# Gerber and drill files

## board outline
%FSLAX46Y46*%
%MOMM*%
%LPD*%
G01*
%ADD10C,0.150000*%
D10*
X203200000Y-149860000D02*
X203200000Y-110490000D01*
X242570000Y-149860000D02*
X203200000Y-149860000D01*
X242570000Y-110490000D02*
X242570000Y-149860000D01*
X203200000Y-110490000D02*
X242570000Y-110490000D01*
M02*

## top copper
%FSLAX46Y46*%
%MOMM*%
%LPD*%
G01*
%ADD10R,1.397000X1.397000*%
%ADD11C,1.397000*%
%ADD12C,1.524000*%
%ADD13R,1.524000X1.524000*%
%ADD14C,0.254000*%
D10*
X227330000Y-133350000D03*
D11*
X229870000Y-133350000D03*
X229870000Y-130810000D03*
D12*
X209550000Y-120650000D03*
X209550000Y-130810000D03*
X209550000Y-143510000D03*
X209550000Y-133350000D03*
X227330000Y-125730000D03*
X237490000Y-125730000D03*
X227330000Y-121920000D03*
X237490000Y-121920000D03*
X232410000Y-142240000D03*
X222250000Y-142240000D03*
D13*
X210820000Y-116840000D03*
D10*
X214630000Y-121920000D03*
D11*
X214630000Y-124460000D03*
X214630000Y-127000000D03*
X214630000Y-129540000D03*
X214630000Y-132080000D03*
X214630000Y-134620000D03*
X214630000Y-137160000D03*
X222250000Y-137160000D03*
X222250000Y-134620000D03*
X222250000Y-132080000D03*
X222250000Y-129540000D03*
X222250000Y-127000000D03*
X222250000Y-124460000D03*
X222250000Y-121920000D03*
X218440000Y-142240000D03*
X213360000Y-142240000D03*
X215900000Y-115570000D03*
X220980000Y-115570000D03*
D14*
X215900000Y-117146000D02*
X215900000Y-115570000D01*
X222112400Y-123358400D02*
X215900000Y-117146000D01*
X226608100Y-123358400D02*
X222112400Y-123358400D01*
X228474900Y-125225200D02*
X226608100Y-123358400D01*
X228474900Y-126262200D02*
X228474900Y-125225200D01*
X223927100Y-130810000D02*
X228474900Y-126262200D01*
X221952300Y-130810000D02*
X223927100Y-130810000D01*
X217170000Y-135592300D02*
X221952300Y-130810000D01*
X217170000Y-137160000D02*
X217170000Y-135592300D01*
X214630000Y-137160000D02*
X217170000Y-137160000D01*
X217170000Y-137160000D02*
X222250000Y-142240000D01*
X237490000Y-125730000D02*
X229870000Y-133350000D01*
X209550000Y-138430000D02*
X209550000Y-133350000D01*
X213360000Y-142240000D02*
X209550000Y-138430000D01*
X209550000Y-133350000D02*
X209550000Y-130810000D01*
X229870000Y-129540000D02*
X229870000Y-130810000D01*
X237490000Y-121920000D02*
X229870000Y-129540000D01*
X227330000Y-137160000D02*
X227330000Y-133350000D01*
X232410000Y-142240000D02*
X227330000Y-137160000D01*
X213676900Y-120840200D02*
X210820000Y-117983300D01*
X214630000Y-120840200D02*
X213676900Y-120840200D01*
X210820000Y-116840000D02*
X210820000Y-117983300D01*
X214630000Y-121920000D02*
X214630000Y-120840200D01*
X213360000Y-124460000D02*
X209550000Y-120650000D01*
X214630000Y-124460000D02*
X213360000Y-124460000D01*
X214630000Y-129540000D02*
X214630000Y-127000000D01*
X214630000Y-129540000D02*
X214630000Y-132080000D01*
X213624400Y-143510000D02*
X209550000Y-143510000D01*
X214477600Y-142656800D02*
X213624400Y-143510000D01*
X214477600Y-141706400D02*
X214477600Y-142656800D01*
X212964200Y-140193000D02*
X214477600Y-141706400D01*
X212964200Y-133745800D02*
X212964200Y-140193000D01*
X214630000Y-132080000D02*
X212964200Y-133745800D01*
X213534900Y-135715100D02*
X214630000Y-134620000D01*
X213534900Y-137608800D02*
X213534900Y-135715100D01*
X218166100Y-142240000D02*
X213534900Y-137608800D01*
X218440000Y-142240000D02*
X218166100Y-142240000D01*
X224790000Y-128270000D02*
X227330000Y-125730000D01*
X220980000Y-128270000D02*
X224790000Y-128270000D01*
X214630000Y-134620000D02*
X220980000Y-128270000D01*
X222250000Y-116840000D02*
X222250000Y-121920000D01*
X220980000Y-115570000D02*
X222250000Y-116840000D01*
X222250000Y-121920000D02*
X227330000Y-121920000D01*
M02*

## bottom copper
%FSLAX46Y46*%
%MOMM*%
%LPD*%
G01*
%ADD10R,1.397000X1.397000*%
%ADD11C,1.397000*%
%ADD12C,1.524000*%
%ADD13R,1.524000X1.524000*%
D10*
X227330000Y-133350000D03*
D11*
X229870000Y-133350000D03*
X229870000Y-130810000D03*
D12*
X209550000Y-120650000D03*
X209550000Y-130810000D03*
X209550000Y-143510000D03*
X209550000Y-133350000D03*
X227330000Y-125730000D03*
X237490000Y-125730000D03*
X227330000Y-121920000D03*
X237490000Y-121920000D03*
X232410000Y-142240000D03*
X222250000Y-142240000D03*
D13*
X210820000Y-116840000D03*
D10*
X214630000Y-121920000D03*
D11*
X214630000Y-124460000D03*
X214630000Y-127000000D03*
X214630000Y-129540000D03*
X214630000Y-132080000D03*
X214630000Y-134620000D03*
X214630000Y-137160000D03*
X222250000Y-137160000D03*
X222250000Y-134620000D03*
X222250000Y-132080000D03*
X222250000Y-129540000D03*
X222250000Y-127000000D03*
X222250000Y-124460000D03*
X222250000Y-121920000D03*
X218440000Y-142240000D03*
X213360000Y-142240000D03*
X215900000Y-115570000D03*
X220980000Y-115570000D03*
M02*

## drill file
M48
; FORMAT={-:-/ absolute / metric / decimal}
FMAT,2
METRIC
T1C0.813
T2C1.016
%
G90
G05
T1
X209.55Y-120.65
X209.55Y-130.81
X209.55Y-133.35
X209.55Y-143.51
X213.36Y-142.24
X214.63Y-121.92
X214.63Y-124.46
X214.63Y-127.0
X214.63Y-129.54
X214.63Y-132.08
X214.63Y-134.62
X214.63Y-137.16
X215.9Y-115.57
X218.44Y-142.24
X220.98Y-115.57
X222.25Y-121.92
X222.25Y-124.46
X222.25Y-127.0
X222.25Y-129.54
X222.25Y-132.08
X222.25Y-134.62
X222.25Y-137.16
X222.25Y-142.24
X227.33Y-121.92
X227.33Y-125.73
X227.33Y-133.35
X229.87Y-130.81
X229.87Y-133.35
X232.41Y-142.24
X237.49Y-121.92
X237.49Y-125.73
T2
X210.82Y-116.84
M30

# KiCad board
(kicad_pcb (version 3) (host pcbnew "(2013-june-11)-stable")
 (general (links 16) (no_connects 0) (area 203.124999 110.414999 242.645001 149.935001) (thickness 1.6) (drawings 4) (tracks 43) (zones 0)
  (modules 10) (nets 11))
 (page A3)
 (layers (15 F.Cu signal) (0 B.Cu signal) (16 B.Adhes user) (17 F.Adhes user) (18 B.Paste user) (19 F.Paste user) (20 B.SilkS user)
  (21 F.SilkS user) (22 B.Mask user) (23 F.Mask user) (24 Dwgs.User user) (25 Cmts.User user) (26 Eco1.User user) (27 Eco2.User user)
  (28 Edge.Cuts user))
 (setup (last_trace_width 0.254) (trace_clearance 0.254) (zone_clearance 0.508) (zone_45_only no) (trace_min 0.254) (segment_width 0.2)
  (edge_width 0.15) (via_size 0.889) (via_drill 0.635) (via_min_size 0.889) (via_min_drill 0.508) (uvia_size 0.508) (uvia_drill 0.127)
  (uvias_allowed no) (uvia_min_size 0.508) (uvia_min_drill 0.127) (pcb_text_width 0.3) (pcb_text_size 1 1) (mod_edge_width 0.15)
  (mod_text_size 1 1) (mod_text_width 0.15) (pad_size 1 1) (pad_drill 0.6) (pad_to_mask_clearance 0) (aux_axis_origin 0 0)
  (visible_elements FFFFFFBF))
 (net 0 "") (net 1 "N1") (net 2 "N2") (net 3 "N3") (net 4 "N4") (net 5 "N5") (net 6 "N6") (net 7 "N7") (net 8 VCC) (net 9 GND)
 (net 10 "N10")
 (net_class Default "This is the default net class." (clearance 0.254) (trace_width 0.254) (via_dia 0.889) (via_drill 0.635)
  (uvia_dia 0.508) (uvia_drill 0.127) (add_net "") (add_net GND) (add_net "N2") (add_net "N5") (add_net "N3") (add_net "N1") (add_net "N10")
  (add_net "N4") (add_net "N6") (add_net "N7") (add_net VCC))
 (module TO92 (layer F.Cu) (at 228.6 132.08 180)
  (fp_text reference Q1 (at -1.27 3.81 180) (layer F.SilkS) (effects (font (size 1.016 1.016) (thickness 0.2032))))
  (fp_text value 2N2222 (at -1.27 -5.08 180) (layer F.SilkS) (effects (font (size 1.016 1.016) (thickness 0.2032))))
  (pad 1 thru_hole rect (at 1.27 -1.27 180) (size 1.397 1.397) (drill 0.8128) (layers *.Cu *.Mask F.SilkS) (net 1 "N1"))
  (pad 2 thru_hole circle (at -1.27 -1.27 180) (size 1.397 1.397) (drill 0.8128) (layers *.Cu *.Mask F.SilkS) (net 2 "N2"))
  (pad 3 thru_hole circle (at -1.27 1.27 180) (size 1.397 1.397) (drill 0.8128) (layers *.Cu *.Mask F.SilkS) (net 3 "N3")))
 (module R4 (layer F.Cu) (at 209.55 125.73 270) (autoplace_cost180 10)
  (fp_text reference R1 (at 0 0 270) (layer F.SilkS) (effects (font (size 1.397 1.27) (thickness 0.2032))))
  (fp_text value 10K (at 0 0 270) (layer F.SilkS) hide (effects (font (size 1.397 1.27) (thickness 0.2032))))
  (pad 1 thru_hole circle (at -5.08 0 270) (size 1.524 1.524) (drill 0.8128) (layers *.Cu *.Mask F.SilkS) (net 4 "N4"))
  (pad 2 thru_hole circle (at 5.08 0 270) (size 1.524 1.524) (drill 0.8128) (layers *.Cu *.Mask F.SilkS) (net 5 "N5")))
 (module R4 (layer F.Cu) (at 209.55 138.43 90) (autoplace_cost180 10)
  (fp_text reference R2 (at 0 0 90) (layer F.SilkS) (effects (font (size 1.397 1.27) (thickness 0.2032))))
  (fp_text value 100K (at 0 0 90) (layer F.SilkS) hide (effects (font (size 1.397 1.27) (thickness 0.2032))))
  (pad 1 thru_hole circle (at -5.08 0 90) (size 1.524 1.524) (drill 0.8128) (layers *.Cu *.Mask F.SilkS) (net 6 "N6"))
  (pad 2 thru_hole circle (at 5.08 0 90) (size 1.524 1.524) (drill 0.8128) (layers *.Cu *.Mask F.SilkS) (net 5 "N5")))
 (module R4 (layer F.Cu) (at 232.41 125.73) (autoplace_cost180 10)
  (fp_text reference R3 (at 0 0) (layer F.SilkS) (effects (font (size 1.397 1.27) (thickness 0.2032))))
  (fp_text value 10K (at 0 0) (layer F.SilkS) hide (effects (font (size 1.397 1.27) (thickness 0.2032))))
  (pad 1 thru_hole circle (at -5.08 0) (size 1.524 1.524) (drill 0.8128) (layers *.Cu *.Mask F.SilkS) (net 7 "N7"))
  (pad 2 thru_hole circle (at 5.08 0) (size 1.524 1.524) (drill 0.8128) (layers *.Cu *.Mask F.SilkS) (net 2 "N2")))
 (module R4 (layer F.Cu) (at 232.41 121.92) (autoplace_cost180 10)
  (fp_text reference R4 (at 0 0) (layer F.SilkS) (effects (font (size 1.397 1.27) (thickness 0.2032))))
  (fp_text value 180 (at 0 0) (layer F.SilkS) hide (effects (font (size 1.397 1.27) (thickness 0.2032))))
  (pad 1 thru_hole circle (at -5.08 0) (size 1.524 1.524) (drill 0.8128) (layers *.Cu *.Mask F.SilkS) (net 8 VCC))
  (pad 2 thru_hole circle (at 5.08 0) (size 1.524 1.524) (drill 0.8128) (layers *.Cu *.Mask F.SilkS) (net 3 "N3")))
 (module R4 (layer F.Cu) (at 227.33 142.24 180) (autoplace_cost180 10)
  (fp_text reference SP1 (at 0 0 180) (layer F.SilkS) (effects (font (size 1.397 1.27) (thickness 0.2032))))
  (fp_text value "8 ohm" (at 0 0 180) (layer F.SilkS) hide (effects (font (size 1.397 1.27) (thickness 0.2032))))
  (pad 1 thru_hole circle (at -5.08 0 180) (size 1.524 1.524) (drill 0.8128) (layers *.Cu *.Mask F.SilkS) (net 1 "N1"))
  (pad 2 thru_hole circle (at 5.08 0 180) (size 1.524 1.524) (drill 0.8128) (layers *.Cu *.Mask F.SilkS) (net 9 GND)))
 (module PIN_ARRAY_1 (layer F.Cu) (at 210.82 116.84)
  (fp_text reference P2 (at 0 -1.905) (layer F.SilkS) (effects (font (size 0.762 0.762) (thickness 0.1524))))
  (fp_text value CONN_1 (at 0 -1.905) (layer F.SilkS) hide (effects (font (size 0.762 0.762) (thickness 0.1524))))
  (pad 1 thru_hole rect (at 0 0) (size 1.524 1.524) (drill 1.016) (layers *.Cu *.Mask F.SilkS) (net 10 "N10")))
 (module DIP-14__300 (layer F.Cu) (at 218.44 129.54 270)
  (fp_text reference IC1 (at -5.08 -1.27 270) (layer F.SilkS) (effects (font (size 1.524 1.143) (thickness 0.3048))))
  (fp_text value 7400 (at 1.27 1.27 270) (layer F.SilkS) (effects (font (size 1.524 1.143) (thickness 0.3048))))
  (pad 1 thru_hole rect (at -7.62 3.81 270) (size 1.397 1.397) (drill 0.8128) (layers *.Cu *.Mask F.SilkS) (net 10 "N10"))
  (pad 2 thru_hole circle (at -5.08 3.81 270) (size 1.397 1.397) (drill 0.8128) (layers *.Cu *.Mask F.SilkS) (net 4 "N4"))
  (pad 3 thru_hole circle (at -2.54 3.81 270) (size 1.397 1.397) (drill 0.8128) (layers *.Cu *.Mask F.SilkS) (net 6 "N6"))
  (pad 4 thru_hole circle (at 0 3.81 270) (size 1.397 1.397) (drill 0.8128) (layers *.Cu *.Mask F.SilkS) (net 6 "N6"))
  (pad 5 thru_hole circle (at 2.54 3.81 270) (size 1.397 1.397) (drill 0.8128) (layers *.Cu *.Mask F.SilkS) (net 6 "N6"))
  (pad 6 thru_hole circle (at 5.08 3.81 270) (size 1.397 1.397) (drill 0.8128) (layers *.Cu *.Mask F.SilkS) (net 7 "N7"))
  (pad 7 thru_hole circle (at 7.62 3.81 270) (size 1.397 1.397) (drill 0.8128) (layers *.Cu *.Mask F.SilkS) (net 9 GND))
  (pad 8 thru_hole circle (at 7.62 -3.81 270) (size 1.397 1.397) (drill 0.8128) (layers *.Cu *.Mask F.SilkS))
  (pad 9 thru_hole circle (at 5.08 -3.81 270) (size 1.397 1.397) (drill 0.8128) (layers *.Cu *.Mask F.SilkS))
  (pad 10 thru_hole circle (at 2.54 -3.81 270) (size 1.397 1.397) (drill 0.8128) (layers *.Cu *.Mask F.SilkS))
  (pad 11 thru_hole circle (at 0 -3.81 270) (size 1.397 1.397) (drill 0.8128) (layers *.Cu *.Mask F.SilkS))
  (pad 12 thru_hole circle (at -2.54 -3.81 270) (size 1.397 1.397) (drill 0.8128) (layers *.Cu *.Mask F.SilkS))
  (pad 13 thru_hole circle (at -5.08 -3.81 270) (size 1.397 1.397) (drill 0.8128) (layers *.Cu *.Mask F.SilkS))
  (pad 14 thru_hole circle (at -7.62 -3.81 270) (size 1.397 1.397) (drill 0.8128) (layers *.Cu *.Mask F.SilkS) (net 8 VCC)))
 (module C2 (layer F.Cu) (at 215.9 142.24 180)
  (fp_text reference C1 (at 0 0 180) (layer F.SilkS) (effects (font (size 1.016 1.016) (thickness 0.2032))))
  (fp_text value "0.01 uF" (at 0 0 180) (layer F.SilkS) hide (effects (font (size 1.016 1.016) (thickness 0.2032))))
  (pad 1 thru_hole circle (at -2.54 0 180) (size 1.397 1.397) (drill 0.8128) (layers *.Cu *.Mask F.SilkS) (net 7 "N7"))
  (pad 2 thru_hole circle (at 2.54 0 180) (size 1.397 1.397) (drill 0.8128) (layers *.Cu *.Mask F.SilkS) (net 5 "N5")))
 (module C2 (layer F.Cu) (at 218.44 115.57)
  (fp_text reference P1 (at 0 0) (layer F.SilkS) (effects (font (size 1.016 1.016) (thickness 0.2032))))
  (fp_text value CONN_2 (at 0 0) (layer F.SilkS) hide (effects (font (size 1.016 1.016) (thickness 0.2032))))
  (pad 1 thru_hole circle (at -2.54 0) (size 1.397 1.397) (drill 0.8128) (layers *.Cu *.Mask F.SilkS) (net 9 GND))
  (pad 2 thru_hole circle (at 2.54 0) (size 1.397 1.397) (drill 0.8128) (layers *.Cu *.Mask F.SilkS) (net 8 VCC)))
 (gr_line (start 203.2 149.86) (end 203.2 110.49) (angle 90) (layer Edge.Cuts) (width 0.15))
 (gr_line (start 242.57 149.86) (end 203.2 149.86) (angle 90) (layer Edge.Cuts) (width 0.15))
 (gr_line (start 242.57 110.49) (end 242.57 149.86) (angle 90) (layer Edge.Cuts) (width 0.15))
 (gr_line (start 203.2 110.49) (end 242.57 110.49) (angle 90) (layer Edge.Cuts) (width 0.15))
 (segment (start 215.9 117.146) (end 215.9 115.57) (width 0.254) (layer F.Cu) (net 9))
 (segment (start 222.1124 123.3584) (end 215.9 117.146) (width 0.254) (layer F.Cu) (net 9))
 (segment (start 226.6081 123.3584) (end 222.1124 123.3584) (width 0.254) (layer F.Cu) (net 9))
 (segment (start 228.4749 125.2252) (end 226.6081 123.3584) (width 0.254) (layer F.Cu) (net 9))
 (segment (start 228.4749 126.2622) (end 228.4749 125.2252) (width 0.254) (layer F.Cu) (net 9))
 (segment (start 223.9271 130.81) (end 228.4749 126.2622) (width 0.254) (layer F.Cu) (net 9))
 (segment (start 221.9523 130.81) (end 223.9271 130.81) (width 0.254) (layer F.Cu) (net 9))
 (segment (start 217.17 135.5923) (end 221.9523 130.81) (width 0.254) (layer F.Cu) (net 9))
 (segment (start 217.17 137.16) (end 217.17 135.5923) (width 0.254) (layer F.Cu) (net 9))
 (segment (start 214.63 137.16) (end 217.17 137.16) (width 0.254) (layer F.Cu) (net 9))
 (segment (start 217.17 137.16) (end 222.25 142.24) (width 0.254) (layer F.Cu) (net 9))
 (segment (start 237.49 125.73) (end 229.87 133.35) (width 0.254) (layer F.Cu) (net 2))
 (segment (start 209.55 138.43) (end 209.55 133.35) (width 0.254) (layer F.Cu) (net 5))
 (segment (start 213.36 142.24) (end 209.55 138.43) (width 0.254) (layer F.Cu) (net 5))
 (segment (start 209.55 133.35) (end 209.55 130.81) (width 0.254) (layer F.Cu) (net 5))
 (segment (start 229.87 129.54) (end 229.87 130.81) (width 0.254) (layer F.Cu) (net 3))
 (segment (start 237.49 121.92) (end 229.87 129.54) (width 0.254) (layer F.Cu) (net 3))
 (segment (start 227.33 137.16) (end 227.33 133.35) (width 0.254) (layer F.Cu) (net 1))
 (segment (start 232.41 142.24) (end 227.33 137.16) (width 0.254) (layer F.Cu) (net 1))
 (segment (start 213.6769 120.8402) (end 210.82 117.9833) (width 0.254) (layer F.Cu) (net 10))
 (segment (start 214.63 120.8402) (end 213.6769 120.8402) (width 0.254) (layer F.Cu) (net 10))
 (segment (start 210.82 116.84) (end 210.82 117.9833) (width 0.254) (layer F.Cu) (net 10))
 (segment (start 214.63 121.92) (end 214.63 120.8402) (width 0.254) (layer F.Cu) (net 10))
 (segment (start 213.36 124.46) (end 209.55 120.65) (width 0.254) (layer F.Cu) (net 4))
 (segment (start 214.63 124.46) (end 213.36 124.46) (width 0.254) (layer F.Cu) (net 4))
 (segment (start 214.63 129.54) (end 214.63 127) (width 0.254) (layer F.Cu) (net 6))
 (segment (start 214.63 129.54) (end 214.63 132.08) (width 0.254) (layer F.Cu) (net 6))
 (segment (start 213.6244 143.51) (end 209.55 143.51) (width 0.254) (layer F.Cu) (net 6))
 (segment (start 214.4776 142.6568) (end 213.6244 143.51) (width 0.254) (layer F.Cu) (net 6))
 (segment (start 214.4776 141.7064) (end 214.4776 142.6568) (width 0.254) (layer F.Cu) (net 6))
 (segment (start 212.9642 140.193) (end 214.4776 141.7064) (width 0.254) (layer F.Cu) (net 6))
 (segment (start 212.9642 133.7458) (end 212.9642 140.193) (width 0.254) (layer F.Cu) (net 6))
 (segment (start 214.63 132.08) (end 212.9642 133.7458) (width 0.254) (layer F.Cu) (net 6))
 (segment (start 213.5349 135.7151) (end 214.63 134.62) (width 0.254) (layer F.Cu) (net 7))
 (segment (start 213.5349 137.6088) (end 213.5349 135.7151) (width 0.254) (layer F.Cu) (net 7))
 (segment (start 218.1661 142.24) (end 213.5349 137.6088) (width 0.254) (layer F.Cu) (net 7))
 (segment (start 218.44 142.24) (end 218.1661 142.24) (width 0.254) (layer F.Cu) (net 7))
 (segment (start 224.79 128.27) (end 227.33 125.73) (width 0.254) (layer F.Cu) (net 7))
 (segment (start 220.98 128.27) (end 224.79 128.27) (width 0.254) (layer F.Cu) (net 7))
 (segment (start 214.63 134.62) (end 220.98 128.27) (width 0.254) (layer F.Cu) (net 7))
 (segment (start 222.25 116.84) (end 222.25 121.92) (width 0.254) (layer F.Cu) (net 8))
 (segment (start 220.98 115.57) (end 222.25 116.84) (width 0.254) (layer F.Cu) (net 8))
 (segment (start 222.25 121.92) (end 227.33 121.92) (width 0.254) (layer F.Cu) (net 8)))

